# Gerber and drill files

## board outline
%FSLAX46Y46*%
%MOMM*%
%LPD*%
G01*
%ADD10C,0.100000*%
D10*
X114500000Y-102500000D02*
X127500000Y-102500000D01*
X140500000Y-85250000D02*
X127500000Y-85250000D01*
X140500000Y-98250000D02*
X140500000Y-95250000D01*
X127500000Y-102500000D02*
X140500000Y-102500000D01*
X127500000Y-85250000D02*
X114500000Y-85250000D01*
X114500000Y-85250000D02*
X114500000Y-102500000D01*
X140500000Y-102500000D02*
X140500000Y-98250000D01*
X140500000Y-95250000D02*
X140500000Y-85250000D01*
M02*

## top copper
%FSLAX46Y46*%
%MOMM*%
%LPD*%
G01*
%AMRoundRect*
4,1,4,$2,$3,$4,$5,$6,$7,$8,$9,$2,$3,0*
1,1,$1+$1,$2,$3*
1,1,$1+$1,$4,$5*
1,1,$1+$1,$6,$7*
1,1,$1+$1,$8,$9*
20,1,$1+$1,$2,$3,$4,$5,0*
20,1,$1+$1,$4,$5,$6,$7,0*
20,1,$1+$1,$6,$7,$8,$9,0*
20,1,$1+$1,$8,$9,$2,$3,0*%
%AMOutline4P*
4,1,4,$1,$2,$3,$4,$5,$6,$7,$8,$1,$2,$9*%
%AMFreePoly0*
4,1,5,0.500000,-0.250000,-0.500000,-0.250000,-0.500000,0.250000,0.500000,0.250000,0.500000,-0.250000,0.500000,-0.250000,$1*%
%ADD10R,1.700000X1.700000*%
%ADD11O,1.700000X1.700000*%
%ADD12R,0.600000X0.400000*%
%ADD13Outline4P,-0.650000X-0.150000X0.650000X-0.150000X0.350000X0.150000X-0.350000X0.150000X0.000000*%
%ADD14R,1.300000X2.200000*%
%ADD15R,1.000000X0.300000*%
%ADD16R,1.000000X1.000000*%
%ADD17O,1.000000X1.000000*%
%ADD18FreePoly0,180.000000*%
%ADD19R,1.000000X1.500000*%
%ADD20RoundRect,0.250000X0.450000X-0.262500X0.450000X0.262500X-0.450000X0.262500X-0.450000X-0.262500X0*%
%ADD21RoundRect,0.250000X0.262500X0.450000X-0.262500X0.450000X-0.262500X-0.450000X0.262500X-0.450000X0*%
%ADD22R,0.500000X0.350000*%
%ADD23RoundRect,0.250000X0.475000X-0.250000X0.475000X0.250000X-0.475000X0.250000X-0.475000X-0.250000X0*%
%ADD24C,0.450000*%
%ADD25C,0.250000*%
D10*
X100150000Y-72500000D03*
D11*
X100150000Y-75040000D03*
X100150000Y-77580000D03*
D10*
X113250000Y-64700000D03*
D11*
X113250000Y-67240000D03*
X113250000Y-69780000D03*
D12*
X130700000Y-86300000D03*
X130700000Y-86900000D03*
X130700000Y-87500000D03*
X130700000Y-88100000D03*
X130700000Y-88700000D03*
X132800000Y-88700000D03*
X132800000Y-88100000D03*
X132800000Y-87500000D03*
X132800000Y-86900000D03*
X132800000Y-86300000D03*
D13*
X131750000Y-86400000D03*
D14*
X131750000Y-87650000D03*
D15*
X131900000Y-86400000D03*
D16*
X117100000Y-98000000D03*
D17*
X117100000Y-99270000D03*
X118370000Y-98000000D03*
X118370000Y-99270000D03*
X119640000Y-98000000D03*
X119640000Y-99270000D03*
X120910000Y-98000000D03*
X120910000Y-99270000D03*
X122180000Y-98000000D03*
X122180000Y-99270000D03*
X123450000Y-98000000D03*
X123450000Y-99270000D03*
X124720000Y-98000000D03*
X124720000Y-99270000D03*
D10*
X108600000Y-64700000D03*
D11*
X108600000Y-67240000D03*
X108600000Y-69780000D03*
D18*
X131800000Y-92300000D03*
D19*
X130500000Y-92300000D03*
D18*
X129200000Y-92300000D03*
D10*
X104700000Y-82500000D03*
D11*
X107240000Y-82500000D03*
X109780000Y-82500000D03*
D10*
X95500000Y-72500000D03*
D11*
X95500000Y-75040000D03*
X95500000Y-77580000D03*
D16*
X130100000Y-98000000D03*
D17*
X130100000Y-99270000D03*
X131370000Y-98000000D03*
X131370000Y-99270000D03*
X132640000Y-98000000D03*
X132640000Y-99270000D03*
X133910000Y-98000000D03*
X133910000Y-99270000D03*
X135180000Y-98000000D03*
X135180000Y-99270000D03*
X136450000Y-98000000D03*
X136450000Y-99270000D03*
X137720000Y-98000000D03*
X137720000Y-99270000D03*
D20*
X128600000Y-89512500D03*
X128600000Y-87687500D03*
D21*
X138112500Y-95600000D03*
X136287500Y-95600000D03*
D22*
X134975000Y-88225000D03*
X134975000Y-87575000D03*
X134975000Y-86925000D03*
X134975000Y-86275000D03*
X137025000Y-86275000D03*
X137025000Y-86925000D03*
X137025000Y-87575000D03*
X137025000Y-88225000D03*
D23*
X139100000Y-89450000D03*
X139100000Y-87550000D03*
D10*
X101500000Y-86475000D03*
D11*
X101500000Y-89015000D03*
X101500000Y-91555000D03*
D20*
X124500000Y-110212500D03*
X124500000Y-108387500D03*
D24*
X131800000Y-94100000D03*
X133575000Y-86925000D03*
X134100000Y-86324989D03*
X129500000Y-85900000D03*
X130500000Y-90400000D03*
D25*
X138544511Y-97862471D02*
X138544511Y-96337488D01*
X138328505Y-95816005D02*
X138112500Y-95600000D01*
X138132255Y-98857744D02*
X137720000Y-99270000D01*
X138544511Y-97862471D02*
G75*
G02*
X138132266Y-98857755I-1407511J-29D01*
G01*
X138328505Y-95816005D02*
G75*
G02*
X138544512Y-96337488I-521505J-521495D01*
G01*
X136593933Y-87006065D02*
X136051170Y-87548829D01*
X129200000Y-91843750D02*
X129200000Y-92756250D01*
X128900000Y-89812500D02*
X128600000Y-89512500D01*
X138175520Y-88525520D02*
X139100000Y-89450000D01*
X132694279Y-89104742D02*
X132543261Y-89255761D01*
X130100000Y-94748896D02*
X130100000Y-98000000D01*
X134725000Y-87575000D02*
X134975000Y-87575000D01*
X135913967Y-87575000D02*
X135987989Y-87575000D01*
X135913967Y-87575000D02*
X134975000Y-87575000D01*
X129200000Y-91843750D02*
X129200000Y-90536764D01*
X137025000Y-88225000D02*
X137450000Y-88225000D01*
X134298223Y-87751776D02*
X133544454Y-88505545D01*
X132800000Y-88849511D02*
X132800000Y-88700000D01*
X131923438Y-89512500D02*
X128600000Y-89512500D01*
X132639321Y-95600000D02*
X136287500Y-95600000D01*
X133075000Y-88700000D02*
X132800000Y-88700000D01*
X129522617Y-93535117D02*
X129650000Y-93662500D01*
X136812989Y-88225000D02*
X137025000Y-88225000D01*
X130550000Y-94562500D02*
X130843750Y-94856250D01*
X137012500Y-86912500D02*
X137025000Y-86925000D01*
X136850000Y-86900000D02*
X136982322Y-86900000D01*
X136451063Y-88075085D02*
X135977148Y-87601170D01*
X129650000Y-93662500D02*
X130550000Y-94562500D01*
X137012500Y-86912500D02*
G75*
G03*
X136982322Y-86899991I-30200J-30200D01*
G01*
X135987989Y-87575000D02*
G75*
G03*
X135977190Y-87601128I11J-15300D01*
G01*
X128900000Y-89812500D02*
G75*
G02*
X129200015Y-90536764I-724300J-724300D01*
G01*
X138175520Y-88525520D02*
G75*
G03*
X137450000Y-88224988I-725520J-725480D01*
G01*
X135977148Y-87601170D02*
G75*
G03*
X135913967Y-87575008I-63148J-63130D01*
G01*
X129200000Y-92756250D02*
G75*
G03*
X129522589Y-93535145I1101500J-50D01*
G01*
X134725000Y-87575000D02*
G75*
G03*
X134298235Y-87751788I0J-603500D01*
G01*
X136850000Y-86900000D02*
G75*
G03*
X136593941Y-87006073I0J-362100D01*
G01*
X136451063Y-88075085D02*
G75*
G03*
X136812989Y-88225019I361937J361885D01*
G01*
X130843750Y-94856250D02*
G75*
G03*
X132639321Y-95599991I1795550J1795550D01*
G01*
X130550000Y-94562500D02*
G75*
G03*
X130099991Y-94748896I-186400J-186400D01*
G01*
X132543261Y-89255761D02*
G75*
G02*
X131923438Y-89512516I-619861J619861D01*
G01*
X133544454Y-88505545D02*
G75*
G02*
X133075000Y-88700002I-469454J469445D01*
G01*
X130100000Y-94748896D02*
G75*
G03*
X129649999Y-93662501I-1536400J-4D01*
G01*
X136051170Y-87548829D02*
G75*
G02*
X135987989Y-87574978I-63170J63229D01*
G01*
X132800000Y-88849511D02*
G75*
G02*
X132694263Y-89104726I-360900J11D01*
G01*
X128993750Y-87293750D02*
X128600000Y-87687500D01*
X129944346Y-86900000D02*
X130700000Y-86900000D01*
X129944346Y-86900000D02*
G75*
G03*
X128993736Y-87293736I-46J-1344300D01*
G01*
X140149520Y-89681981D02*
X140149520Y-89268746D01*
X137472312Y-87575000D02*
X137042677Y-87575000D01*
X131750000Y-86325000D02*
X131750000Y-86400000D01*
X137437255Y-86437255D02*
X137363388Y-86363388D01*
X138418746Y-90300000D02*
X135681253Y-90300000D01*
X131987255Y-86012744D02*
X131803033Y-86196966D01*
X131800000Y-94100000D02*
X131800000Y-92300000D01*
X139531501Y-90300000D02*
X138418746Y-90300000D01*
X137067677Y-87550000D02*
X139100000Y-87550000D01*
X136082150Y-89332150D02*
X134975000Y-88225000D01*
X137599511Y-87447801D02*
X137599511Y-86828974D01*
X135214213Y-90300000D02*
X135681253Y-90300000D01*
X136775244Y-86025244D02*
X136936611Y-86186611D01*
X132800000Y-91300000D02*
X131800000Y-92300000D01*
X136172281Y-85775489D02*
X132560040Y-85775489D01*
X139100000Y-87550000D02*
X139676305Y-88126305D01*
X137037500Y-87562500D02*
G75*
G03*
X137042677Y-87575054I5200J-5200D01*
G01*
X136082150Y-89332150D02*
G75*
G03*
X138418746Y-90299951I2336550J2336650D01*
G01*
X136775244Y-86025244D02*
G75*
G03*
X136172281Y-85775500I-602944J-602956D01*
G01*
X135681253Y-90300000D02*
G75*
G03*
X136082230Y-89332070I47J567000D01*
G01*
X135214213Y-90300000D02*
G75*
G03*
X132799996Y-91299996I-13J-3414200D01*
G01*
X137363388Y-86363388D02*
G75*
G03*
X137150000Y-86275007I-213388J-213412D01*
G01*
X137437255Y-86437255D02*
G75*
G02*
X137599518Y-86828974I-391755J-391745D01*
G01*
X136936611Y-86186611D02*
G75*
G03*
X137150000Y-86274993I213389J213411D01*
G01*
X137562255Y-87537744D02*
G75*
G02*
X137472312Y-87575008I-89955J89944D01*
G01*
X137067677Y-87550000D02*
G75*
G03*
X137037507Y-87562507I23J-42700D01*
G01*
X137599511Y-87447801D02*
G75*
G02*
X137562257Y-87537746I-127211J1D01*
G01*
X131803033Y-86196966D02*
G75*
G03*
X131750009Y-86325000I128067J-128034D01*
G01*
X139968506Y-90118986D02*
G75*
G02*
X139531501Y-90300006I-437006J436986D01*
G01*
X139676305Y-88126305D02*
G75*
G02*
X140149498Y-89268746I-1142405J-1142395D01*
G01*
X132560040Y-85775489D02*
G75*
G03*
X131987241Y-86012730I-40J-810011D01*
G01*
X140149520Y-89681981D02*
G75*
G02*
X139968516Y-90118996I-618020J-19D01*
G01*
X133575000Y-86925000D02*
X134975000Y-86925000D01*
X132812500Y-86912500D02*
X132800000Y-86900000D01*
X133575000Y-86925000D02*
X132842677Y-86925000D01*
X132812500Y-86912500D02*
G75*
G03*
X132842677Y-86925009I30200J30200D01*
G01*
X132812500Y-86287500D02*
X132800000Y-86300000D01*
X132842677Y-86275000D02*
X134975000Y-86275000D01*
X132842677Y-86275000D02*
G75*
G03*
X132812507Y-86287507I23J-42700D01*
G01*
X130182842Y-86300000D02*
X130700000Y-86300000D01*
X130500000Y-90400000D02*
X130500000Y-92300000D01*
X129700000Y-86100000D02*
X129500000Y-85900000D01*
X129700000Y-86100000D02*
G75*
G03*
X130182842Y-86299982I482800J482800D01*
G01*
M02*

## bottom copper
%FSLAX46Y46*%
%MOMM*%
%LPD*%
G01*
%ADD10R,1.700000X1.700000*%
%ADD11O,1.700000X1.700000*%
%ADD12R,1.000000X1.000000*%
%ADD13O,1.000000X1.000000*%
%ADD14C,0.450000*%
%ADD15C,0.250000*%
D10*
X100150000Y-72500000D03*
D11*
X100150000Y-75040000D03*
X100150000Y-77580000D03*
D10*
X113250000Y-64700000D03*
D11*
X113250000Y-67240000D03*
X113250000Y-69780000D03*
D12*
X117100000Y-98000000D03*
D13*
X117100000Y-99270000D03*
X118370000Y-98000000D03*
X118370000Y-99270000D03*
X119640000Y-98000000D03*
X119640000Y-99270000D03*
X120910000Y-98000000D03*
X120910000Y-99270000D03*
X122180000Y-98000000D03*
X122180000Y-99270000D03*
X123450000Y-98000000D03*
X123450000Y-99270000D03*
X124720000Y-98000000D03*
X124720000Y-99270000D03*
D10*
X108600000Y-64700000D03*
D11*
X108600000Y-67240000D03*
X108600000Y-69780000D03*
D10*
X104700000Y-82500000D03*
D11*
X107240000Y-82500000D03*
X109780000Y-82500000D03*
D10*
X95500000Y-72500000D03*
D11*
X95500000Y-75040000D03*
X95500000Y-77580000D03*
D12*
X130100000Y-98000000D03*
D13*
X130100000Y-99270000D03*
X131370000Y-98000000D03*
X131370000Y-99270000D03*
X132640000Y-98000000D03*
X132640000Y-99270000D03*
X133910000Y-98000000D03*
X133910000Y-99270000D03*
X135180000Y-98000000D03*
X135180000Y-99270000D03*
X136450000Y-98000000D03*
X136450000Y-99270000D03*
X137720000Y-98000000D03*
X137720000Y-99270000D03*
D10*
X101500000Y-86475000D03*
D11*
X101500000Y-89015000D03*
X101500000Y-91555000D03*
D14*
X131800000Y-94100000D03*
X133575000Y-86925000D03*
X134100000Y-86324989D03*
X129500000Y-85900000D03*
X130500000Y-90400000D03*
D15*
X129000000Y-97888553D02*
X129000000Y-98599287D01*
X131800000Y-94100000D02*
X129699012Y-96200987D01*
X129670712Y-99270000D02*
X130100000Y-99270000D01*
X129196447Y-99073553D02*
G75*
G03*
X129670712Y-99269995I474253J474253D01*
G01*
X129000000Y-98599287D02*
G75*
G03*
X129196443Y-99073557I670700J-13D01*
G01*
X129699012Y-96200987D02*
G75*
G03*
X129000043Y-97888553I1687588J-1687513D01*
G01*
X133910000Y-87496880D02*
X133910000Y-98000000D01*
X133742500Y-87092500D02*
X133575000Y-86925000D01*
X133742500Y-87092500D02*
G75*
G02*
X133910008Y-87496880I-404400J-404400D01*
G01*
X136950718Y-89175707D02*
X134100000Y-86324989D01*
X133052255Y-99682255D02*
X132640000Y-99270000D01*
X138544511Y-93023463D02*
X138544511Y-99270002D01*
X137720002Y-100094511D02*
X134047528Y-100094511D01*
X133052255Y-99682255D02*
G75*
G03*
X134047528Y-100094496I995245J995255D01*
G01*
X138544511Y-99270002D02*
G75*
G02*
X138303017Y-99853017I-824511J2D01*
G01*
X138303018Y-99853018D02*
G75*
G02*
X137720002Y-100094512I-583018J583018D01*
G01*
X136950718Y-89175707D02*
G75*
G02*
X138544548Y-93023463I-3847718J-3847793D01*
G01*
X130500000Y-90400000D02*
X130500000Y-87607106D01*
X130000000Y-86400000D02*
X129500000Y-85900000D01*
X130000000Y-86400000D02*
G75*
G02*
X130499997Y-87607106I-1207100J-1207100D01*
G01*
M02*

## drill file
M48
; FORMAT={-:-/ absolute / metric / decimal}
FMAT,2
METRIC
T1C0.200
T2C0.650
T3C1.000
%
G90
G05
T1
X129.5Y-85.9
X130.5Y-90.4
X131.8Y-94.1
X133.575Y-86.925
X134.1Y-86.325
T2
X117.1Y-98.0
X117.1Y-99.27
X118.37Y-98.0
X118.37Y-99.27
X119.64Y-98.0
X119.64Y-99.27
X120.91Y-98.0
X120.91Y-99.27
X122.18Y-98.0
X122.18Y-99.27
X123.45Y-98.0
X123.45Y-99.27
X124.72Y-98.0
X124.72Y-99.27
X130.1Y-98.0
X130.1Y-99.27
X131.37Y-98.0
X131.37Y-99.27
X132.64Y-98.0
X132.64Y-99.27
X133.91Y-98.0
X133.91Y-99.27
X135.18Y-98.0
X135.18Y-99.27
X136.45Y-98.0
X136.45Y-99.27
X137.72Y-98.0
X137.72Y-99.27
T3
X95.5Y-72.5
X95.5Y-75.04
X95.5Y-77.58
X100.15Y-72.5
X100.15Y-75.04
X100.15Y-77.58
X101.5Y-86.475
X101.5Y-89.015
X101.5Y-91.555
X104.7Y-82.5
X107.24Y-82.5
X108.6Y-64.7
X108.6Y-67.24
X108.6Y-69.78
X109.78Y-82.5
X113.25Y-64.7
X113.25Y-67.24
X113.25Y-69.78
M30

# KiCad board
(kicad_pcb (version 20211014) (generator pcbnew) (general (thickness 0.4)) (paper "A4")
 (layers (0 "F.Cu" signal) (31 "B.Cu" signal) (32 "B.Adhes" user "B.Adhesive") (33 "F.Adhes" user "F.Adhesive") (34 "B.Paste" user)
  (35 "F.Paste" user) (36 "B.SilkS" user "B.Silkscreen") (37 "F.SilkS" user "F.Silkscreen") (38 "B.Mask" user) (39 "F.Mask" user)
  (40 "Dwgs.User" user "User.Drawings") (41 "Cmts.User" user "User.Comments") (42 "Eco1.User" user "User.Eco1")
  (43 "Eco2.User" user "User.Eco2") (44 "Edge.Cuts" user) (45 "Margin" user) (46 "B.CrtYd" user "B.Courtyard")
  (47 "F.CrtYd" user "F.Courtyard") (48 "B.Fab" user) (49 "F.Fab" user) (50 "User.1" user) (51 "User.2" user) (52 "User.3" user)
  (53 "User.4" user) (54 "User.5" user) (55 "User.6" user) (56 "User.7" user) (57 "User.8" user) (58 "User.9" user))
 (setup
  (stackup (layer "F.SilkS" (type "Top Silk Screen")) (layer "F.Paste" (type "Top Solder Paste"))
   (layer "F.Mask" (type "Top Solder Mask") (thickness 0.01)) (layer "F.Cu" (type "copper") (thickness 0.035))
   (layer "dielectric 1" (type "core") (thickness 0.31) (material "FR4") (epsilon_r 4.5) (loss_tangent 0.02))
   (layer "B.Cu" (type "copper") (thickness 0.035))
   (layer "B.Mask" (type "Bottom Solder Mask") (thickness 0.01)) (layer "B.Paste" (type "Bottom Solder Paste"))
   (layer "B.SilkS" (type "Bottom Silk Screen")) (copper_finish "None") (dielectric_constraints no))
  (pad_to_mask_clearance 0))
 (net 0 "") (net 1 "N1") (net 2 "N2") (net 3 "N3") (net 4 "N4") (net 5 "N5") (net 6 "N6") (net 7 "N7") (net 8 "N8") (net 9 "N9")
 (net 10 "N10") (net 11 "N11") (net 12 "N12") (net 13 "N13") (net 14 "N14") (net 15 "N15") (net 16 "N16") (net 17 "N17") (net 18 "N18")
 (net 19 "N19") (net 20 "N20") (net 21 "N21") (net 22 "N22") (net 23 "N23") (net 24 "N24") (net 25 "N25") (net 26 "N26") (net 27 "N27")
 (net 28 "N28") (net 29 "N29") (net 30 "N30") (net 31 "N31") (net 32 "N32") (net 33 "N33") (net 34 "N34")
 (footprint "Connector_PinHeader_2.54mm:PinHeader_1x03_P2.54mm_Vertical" (layer "F.Cu") (at 100.15 72.5)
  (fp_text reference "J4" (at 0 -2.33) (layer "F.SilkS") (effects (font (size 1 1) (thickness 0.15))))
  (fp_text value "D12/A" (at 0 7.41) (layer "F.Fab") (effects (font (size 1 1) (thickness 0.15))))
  (pad "1" thru_hole rect (at 0 0) (size 1.7 1.7) (drill 1) (layers *.Cu *.Mask) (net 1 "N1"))
  (pad "2" thru_hole oval (at 0 2.54) (size 1.7 1.7) (drill 1) (layers *.Cu *.Mask) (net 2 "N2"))
  (pad "3" thru_hole oval (at 0 5.08) (size 1.7 1.7) (drill 1) (layers *.Cu *.Mask) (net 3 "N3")))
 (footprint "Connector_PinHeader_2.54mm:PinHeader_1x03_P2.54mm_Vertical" (layer "F.Cu") (at 113.25 64.7)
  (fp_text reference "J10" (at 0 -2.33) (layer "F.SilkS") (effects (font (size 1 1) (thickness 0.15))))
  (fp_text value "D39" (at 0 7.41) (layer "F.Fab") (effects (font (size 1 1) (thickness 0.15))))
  (pad "1" thru_hole rect (at 0 0) (size 1.7 1.7) (drill 1) (layers *.Cu *.Mask) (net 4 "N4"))
  (pad "2" thru_hole oval (at 0 2.54) (size 1.7 1.7) (drill 1) (layers *.Cu *.Mask) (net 2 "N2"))
  (pad "3" thru_hole oval (at 0 5.08) (size 1.7 1.7) (drill 1) (layers *.Cu *.Mask) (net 3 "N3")))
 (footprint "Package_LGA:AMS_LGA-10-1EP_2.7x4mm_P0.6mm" (layer "F.Cu") (at 131.75 87.5)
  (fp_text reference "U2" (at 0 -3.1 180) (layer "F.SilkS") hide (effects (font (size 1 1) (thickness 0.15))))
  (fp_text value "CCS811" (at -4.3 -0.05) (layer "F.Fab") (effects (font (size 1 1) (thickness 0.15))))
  (pad "1" smd rect (at -1.05 -1.2) (size 0.6 0.4) (layers "F.Cu" "F.Paste" "F.Mask") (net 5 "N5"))
  (pad "2" smd rect (at -1.05 -0.6) (size 0.6 0.4) (layers "F.Cu" "F.Paste" "F.Mask") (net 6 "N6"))
  (pad "3" smd rect (at -1.05 0) (size 0.6 0.4) (layers "F.Cu" "F.Paste" "F.Mask") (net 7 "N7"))
  (pad "4" smd rect (at -1.05 0.6) (size 0.6 0.4) (layers "F.Cu" "F.Paste" "F.Mask") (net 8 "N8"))
  (pad "5" smd rect (at -1.05 1.2) (size 0.6 0.4) (layers "F.Cu" "F.Paste" "F.Mask") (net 8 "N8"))
  (pad "6" smd rect (at 1.05 1.2) (size 0.6 0.4) (layers "F.Cu" "F.Paste" "F.Mask") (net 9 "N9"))
  (pad "7" smd rect (at 1.05 0.6) (size 0.6 0.4) (layers "F.Cu" "F.Paste" "F.Mask") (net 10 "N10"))
  (pad "8" smd rect (at 1.05 0) (size 0.6 0.4) (layers "F.Cu" "F.Paste" "F.Mask") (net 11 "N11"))
  (pad "9" smd rect (at 1.05 -0.6) (size 0.6 0.4) (layers "F.Cu" "F.Paste" "F.Mask") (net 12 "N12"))
  (pad "10" smd rect (at 1.05 -1.2) (size 0.6 0.4) (layers "F.Cu" "F.Paste" "F.Mask") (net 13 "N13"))
  (pad "11" smd trapezoid (at 0 -1.1) (size 1 0.3) (rect_delta 0 0.3) (layers "F.Cu" "F.Paste" "F.Mask") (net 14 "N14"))
  (pad "11" smd rect (at 0 0.15) (size 1.3 2.2) (layers "F.Cu" "F.Paste" "F.Mask") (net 14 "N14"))
  (pad "11" smd rect (at 0.15 -1.1) (size 1 0.3) (layers "F.Cu" "F.Paste" "F.Mask") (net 14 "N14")))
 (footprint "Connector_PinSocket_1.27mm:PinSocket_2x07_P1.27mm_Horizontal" (layer "F.Cu") (at 117.1 98 90)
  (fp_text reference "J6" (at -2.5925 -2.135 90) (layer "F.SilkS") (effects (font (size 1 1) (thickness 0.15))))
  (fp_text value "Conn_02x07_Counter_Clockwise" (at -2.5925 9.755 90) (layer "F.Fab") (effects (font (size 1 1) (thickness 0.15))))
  (pad "1" thru_hole rect (at 0 0 90) (size 1 1) (drill 0.65) (layers *.Cu *.Mask) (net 2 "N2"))
  (pad "2" thru_hole oval (at -1.27 0 90) (size 1 1) (drill 0.65) (layers *.Cu *.Mask) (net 3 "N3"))
  (pad "3" thru_hole oval (at 0 1.27 90) (size 1 1) (drill 0.65) (layers *.Cu *.Mask) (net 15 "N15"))
  (pad "4" thru_hole oval (at -1.27 1.27 90) (size 1 1) (drill 0.65) (layers *.Cu *.Mask) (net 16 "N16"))
  (pad "5" thru_hole oval (at 0 2.54 90) (size 1 1) (drill 0.65) (layers *.Cu *.Mask) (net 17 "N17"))
  (pad "6" thru_hole oval (at -1.27 2.54 90) (size 1 1) (drill 0.65) (layers *.Cu *.Mask) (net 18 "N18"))
  (pad "7" thru_hole oval (at 0 3.81 90) (size 1 1) (drill 0.65) (layers *.Cu *.Mask) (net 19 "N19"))
  (pad "8" thru_hole oval (at -1.27 3.81 90) (size 1 1) (drill 0.65) (layers *.Cu *.Mask) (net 4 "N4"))
  (pad "9" thru_hole oval (at 0 5.08 90) (size 1 1) (drill 0.65) (layers *.Cu *.Mask) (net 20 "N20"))
  (pad "10" thru_hole oval (at -1.27 5.08 90) (size 1 1) (drill 0.65) (layers *.Cu *.Mask) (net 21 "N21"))
  (pad "11" thru_hole oval (at 0 6.35 90) (size 1 1) (drill 0.65) (layers *.Cu *.Mask) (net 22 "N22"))
  (pad "12" thru_hole oval (at -1.27 6.35 90) (size 1 1) (drill 0.65) (layers *.Cu *.Mask) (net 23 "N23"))
  (pad "13" thru_hole oval (at 0 7.62 90) (size 1 1) (drill 0.65) (layers *.Cu *.Mask) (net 1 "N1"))
  (pad "14" thru_hole oval (at -1.27 7.62 90) (size 1 1) (drill 0.65) (layers *.Cu *.Mask) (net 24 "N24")))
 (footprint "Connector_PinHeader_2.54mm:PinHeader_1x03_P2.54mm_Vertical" (layer "F.Cu") (at 108.6 64.7)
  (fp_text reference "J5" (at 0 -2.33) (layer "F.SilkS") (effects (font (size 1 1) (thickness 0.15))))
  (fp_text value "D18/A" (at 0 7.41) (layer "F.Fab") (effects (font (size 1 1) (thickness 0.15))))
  (pad "1" thru_hole rect (at 0 0) (size 1.7 1.7) (drill 1) (layers *.Cu *.Mask) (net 21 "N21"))
  (pad "2" thru_hole oval (at 0 2.54) (size 1.7 1.7) (drill 1) (layers *.Cu *.Mask) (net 2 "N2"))
  (pad "3" thru_hole oval (at 0 5.08) (size 1.7 1.7) (drill 1) (layers *.Cu *.Mask) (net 3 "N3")))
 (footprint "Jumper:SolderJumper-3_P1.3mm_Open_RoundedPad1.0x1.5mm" (layer "F.Cu") (at 130.5 92.3 180)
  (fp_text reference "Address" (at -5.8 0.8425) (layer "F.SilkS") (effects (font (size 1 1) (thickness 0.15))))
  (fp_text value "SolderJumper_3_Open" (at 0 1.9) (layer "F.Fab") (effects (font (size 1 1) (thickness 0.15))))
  (pad "1" smd custom (at -1.3 0 180) (size 1 0.5) (layers "F.Cu" "F.Mask") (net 14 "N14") (zone_connect 2)
   (options (clearance outline) (anchor rect)) (primitives))
  (pad "2" smd rect (at 0 0 180) (size 1 1.5) (layers "F.Cu" "F.Mask") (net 5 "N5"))
  (pad "3" smd custom (at 1.3 0 180) (size 1 0.5) (layers "F.Cu" "F.Mask") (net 9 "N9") (zone_connect 2)
   (options (clearance outline) (anchor rect)) (primitives)))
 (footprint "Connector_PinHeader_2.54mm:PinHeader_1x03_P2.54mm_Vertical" (layer "F.Cu") (at 104.7 82.5 90)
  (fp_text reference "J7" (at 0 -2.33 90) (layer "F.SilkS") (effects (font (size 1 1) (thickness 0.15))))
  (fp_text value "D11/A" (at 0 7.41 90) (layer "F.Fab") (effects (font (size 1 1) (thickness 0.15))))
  (pad "1" thru_hole rect (at 0 0 90) (size 1.7 1.7) (drill 1) (layers *.Cu *.Mask) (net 23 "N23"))
  (pad "2" thru_hole oval (at 0 2.54 90) (size 1.7 1.7) (drill 1) (layers *.Cu *.Mask) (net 2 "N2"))
  (pad "3" thru_hole oval (at 0 5.08 90) (size 1.7 1.7) (drill 1) (layers *.Cu *.Mask) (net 3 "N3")))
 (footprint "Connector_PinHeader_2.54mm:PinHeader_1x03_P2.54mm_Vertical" (layer "F.Cu") (at 95.5 72.5)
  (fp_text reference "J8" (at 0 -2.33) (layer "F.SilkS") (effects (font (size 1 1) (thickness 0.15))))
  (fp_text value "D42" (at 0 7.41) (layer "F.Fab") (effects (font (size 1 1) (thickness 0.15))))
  (pad "1" thru_hole rect (at 0 0) (size 1.7 1.7) (drill 1) (layers *.Cu *.Mask) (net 20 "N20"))
  (pad "2" thru_hole oval (at 0 2.54) (size 1.7 1.7) (drill 1) (layers *.Cu *.Mask) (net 2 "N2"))
  (pad "3" thru_hole oval (at 0 5.08) (size 1.7 1.7) (drill 1) (layers *.Cu *.Mask) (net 3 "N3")))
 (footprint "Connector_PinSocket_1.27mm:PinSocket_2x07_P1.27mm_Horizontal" (layer "F.Cu") (at 130.1 98 90)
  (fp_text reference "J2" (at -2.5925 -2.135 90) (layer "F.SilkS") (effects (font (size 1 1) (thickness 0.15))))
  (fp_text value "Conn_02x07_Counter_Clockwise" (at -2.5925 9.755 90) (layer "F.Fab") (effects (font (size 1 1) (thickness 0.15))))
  (pad "1" thru_hole rect (at 0 0 90) (size 1 1) (drill 0.65) (layers *.Cu *.Mask) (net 9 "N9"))
  (pad "2" thru_hole oval (at -1.27 0 90) (size 1 1) (drill 0.65) (layers *.Cu *.Mask) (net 14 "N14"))
  (pad "3" thru_hole oval (at 0 1.27 90) (size 1 1) (drill 0.65) (layers *.Cu *.Mask) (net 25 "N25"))
  (pad "4" thru_hole oval (at -1.27 1.27 90) (size 1 1) (drill 0.65) (layers *.Cu *.Mask) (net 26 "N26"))
  (pad "5" thru_hole oval (at 0 2.54 90) (size 1 1) (drill 0.65) (layers *.Cu *.Mask) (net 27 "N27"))
  (pad "6" thru_hole oval (at -1.27 2.54 90) (size 1 1) (drill 0.65) (layers *.Cu *.Mask) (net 13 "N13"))
  (pad "7" thru_hole oval (at 0 3.81 90) (size 1 1) (drill 0.65) (layers *.Cu *.Mask) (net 12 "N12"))
  (pad "8" thru_hole oval (at -1.27 3.81 90) (size 1 1) (drill 0.65) (layers *.Cu *.Mask) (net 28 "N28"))
  (pad "9" thru_hole oval (at 0 5.08 90) (size 1 1) (drill 0.65) (layers *.Cu *.Mask) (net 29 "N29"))
  (pad "10" thru_hole oval (at -1.27 5.08 90) (size 1 1) (drill 0.65) (layers *.Cu *.Mask) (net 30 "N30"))
  (pad "11" thru_hole oval (at 0 6.35 90) (size 1 1) (drill 0.65) (layers *.Cu *.Mask) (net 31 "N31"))
  (pad "12" thru_hole oval (at -1.27 6.35 90) (size 1 1) (drill 0.65) (layers *.Cu *.Mask) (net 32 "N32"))
  (pad "13" thru_hole oval (at 0 7.62 90) (size 1 1) (drill 0.65) (layers *.Cu *.Mask) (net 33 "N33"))
  (pad "14" thru_hole oval (at -1.27 7.62 90) (size 1 1) (drill 0.65) (layers *.Cu *.Mask) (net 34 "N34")))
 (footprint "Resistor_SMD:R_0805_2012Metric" (layer "F.Cu") (at 128.6 88.6 90)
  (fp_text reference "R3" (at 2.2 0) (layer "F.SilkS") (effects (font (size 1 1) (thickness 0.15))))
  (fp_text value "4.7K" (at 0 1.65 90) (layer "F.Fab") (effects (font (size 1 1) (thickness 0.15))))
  (pad "1" smd roundrect (at -0.9125 0 90) (size 1.025 1.4) (layers "F.Cu" "F.Paste" "F.Mask") (roundrect_rratio 0.243902) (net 9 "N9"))
  (pad "2" smd roundrect (at 0.9125 0 90) (size 1.025 1.4) (layers "F.Cu" "F.Paste" "F.Mask") (roundrect_rratio 0.243902) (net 6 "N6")))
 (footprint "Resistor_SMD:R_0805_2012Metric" (layer "F.Cu") (at 137.2 95.6 180)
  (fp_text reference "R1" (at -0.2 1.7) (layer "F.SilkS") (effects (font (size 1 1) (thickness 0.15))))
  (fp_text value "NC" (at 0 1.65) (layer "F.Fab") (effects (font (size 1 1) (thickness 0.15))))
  (pad "1" smd roundrect (at -0.9125 0 180) (size 1.025 1.4) (layers "F.Cu" "F.Paste" "F.Mask") (roundrect_rratio 0.243902) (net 34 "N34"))
  (pad "2" smd roundrect (at 0.9125 0 180) (size 1.025 1.4) (layers "F.Cu" "F.Paste" "F.Mask") (roundrect_rratio 0.243902) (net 9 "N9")))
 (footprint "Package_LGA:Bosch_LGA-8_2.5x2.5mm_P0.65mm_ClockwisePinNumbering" (layer "F.Cu") (at 136 87.25 90)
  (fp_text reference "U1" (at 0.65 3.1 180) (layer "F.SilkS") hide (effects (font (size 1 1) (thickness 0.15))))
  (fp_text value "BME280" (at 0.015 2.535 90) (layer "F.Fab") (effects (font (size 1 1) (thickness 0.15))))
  (pad "1" smd rect (at -0.975 -1.025 180) (size 0.5 0.35) (layers "F.Cu" "F.Paste" "F.Mask") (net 14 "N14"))
  (pad "2" smd rect (at -0.325 -1.025 180) (size 0.5 0.35) (layers "F.Cu" "F.Paste" "F.Mask") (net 9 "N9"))
  (pad "3" smd rect (at 0.325 -1.025 180) (size 0.5 0.35) (layers "F.Cu" "F.Paste" "F.Mask") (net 12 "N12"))
  (pad "4" smd rect (at 0.975 -1.025 180) (size 0.5 0.35) (layers "F.Cu" "F.Paste" "F.Mask") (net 13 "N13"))
  (pad "5" smd rect (at 0.975 1.025 180) (size 0.5 0.35) (layers "F.Cu" "F.Paste" "F.Mask") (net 14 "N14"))
  (pad "6" smd rect (at 0.325 1.025 180) (size 0.5 0.35) (layers "F.Cu" "F.Paste" "F.Mask") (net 9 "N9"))
  (pad "7" smd rect (at -0.325 1.025 180) (size 0.5 0.35) (layers "F.Cu" "F.Paste" "F.Mask") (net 14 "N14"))
  (pad "8" smd rect (at -0.975 1.025 180) (size 0.5 0.35) (layers "F.Cu" "F.Paste" "F.Mask") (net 9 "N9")))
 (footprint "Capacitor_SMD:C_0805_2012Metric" (layer "F.Cu") (at 139.1 88.5 90)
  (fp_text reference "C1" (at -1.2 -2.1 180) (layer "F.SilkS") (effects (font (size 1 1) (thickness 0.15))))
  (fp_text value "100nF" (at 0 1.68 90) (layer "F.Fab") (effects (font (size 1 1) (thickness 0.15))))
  (pad "1" smd roundrect (at -0.95 0 90) (size 1 1.45) (layers "F.Cu" "F.Paste" "F.Mask") (roundrect_rratio 0.25) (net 9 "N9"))
  (pad "2" smd roundrect (at 0.95 0 90) (size 1 1.45) (layers "F.Cu" "F.Paste" "F.Mask") (roundrect_rratio 0.25) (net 14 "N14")))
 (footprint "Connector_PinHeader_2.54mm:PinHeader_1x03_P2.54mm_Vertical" (layer "F.Cu") (at 101.5 86.475)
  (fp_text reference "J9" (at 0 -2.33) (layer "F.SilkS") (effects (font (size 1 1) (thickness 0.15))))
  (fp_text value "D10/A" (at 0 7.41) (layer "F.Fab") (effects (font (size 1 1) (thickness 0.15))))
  (pad "1" thru_hole rect (at 0 0) (size 1.7 1.7) (drill 1) (layers *.Cu *.Mask) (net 22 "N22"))
  (pad "2" thru_hole oval (at 0 2.54) (size 1.7 1.7) (drill 1) (layers *.Cu *.Mask) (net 2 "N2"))
  (pad "3" thru_hole oval (at 0 5.08) (size 1.7 1.7) (drill 1) (layers *.Cu *.Mask) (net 3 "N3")))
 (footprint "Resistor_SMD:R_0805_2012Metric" (layer "F.Cu") (at 124.5 109.3 90)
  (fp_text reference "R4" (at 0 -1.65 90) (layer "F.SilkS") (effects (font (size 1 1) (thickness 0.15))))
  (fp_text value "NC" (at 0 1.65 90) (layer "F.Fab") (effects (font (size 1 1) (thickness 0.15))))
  (pad "1" smd roundrect (at -0.9125 0 90) (size 1.025 1.4) (layers "F.Cu" "F.Paste" "F.Mask") (roundrect_rratio 0.243902) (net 24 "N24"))
  (pad "2" smd roundrect (at 0.9125 0 90) (size 1.025 1.4) (layers "F.Cu" "F.Paste" "F.Mask") (roundrect_rratio 0.243902) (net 2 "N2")))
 (gr_line (start 114.5 102.5) (end 127.5 102.5) (layer "Edge.Cuts") (width 0.1))
 (gr_line (start 140.5 85.25) (end 127.5 85.25) (layer "Edge.Cuts") (width 0.1))
 (gr_line (start 140.5 98.25) (end 140.5 95.25) (layer "Edge.Cuts") (width 0.1))
 (gr_line (start 127.5 102.5) (end 140.5 102.5) (layer "Edge.Cuts") (width 0.1))
 (gr_line (start 127.5 85.25) (end 114.5 85.25) (layer "Edge.Cuts") (width 0.1))
 (gr_line (start 114.5 85.25) (end 114.5 102.5) (layer "Edge.Cuts") (width 0.1))
 (gr_line (start 140.5 102.5) (end 140.5 98.25) (layer "Edge.Cuts") (width 0.1))
 (gr_line (start 140.5 95.25) (end 140.5 85.25) (layer "Edge.Cuts") (width 0.1))
 (segment (start 138.544511 97.862471) (end 138.544511 96.337488) (width 0.25) (layer "F.Cu") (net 34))
 (segment (start 138.328505 95.816005) (end 138.1125 95.6) (width 0.25) (layer "F.Cu") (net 34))
 (segment (start 138.132255 98.857744) (end 137.72 99.27) (width 0.25) (layer "F.Cu") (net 34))
 (arc (start 138.544511 97.862471) (mid 138.437369 98.401109) (end 138.132255 98.857744) (width 0.25) (layer "F.Cu") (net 34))
 (arc (start 138.328505 95.816005) (mid 138.488372 96.055263) (end 138.544511 96.337488) (width 0.25) (layer "F.Cu") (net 34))
 (segment (start 136.593933 87.006065) (end 136.05117 87.548829) (width 0.25) (layer "F.Cu") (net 9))
 (segment (start 129.2 91.84375) (end 129.2 92.75625) (width 0.25) (layer "F.Cu") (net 9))
 (segment (start 128.9 89.8125) (end 128.6 89.5125) (width 0.25) (layer "F.Cu") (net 9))
 (segment (start 138.17552 88.52552) (end 139.1 89.45) (width 0.25) (layer "F.Cu") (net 9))
 (segment (start 132.694279 89.104742) (end 132.543261 89.255761) (width 0.25) (layer "F.Cu") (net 9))
 (segment (start 130.1 94.748896) (end 130.1 98) (width 0.25) (layer "F.Cu") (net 9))
 (segment (start 134.725 87.575) (end 134.975 87.575) (width 0.25) (layer "F.Cu") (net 9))
 (segment (start 135.913967 87.575) (end 135.987989 87.575) (width 0.25) (layer "F.Cu") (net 9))
 (segment (start 135.913967 87.575) (end 134.975 87.575) (width 0.25) (layer "F.Cu") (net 9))
 (segment (start 129.2 91.84375) (end 129.2 90.536764) (width 0.25) (layer "F.Cu") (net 9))
 (segment (start 137.025 88.225) (end 137.45 88.225) (width 0.25) (layer "F.Cu") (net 9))
 (segment (start 134.298223 87.751776) (end 133.544454 88.505545) (width 0.25) (layer "F.Cu") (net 9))
 (segment (start 132.8 88.849511) (end 132.8 88.7) (width 0.25) (layer "F.Cu") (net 9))
 (segment (start 131.923438 89.5125) (end 128.6 89.5125) (width 0.25) (layer "F.Cu") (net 9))
 (segment (start 132.639321 95.6) (end 136.2875 95.6) (width 0.25) (layer "F.Cu") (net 9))
 (segment (start 133.075 88.7) (end 132.8 88.7) (width 0.25) (layer "F.Cu") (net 9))
 (segment (start 129.522617 93.535117) (end 129.65 93.6625) (width 0.25) (layer "F.Cu") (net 9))
 (segment (start 136.812989 88.225) (end 137.025 88.225) (width 0.25) (layer "F.Cu") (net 9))
 (segment (start 130.55 94.5625) (end 130.84375 94.85625) (width 0.25) (layer "F.Cu") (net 9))
 (segment (start 137.0125 86.9125) (end 137.025 86.925) (width 0.25) (layer "F.Cu") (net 9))
 (segment (start 136.85 86.9) (end 136.982322 86.9) (width 0.25) (layer "F.Cu") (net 9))
 (segment (start 136.451063 88.075085) (end 135.977148 87.60117) (width 0.25) (layer "F.Cu") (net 9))
 (segment (start 129.65 93.6625) (end 130.55 94.5625) (width 0.25) (layer "F.Cu") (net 9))
 (arc (start 137.0125 86.9125) (mid 136.998654 86.903248) (end 136.982322 86.9) (width 0.25) (layer "F.Cu") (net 9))
 (arc (start 135.987989 87.575) (mid 135.973825 87.584463) (end 135.977148 87.60117) (width 0.25) (layer "F.Cu") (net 9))
 (arc (start 128.9 89.8125) (mid 129.122032 90.144795) (end 129.2 90.536764) (width 0.25) (layer "F.Cu") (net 9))
 (arc (start 138.17552 88.52552) (mid 137.842648 88.303102) (end 137.45 88.225) (width 0.25) (layer "F.Cu") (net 9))
 (arc (start 135.977148 87.60117) (mid 135.94816 87.581801) (end 135.913967 87.575) (width 0.25) (layer "F.Cu") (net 9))
 (arc (start 129.2 92.75625) (mid 129.283845 93.177769) (end 129.522617 93.535117) (width 0.25) (layer "F.Cu") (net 9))
 (arc (start 134.725 87.575) (mid 134.49403 87.620942) (end 134.298223 87.751776) (width 0.25) (layer "F.Cu") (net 9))
 (arc (start 136.85 86.9) (mid 136.711417 86.927565) (end 136.593933 87.006065) (width 0.25) (layer "F.Cu") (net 9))
 (arc (start 136.451063 88.075085) (mid 136.617116 88.186038) (end 136.812989 88.225) (width 0.25) (layer "F.Cu") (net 9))
 (arc (start 130.84375 94.85625) (mid 131.667565 95.406705) (end 132.639321 95.6) (width 0.25) (layer "F.Cu") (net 9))
 (arc (start 130.55 94.5625) (mid 130.262727 94.505357) (end 130.1 94.748896) (width 0.25) (layer "F.Cu") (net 9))
 (arc (start 132.543261 89.255761) (mid 132.258883 89.445775) (end 131.923438 89.5125) (width 0.25) (layer "F.Cu") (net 9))
 (arc (start 133.544454 88.505545) (mid 133.329066 88.649462) (end 133.075 88.7) (width 0.25) (layer "F.Cu") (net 9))
 (arc (start 130.1 94.748896) (mid 129.983048 94.160942) (end 129.65 93.6625) (width 0.25) (layer "F.Cu") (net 9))
 (arc (start 136.05117 87.548829) (mid 136.022182 87.568198) (end 135.987989 87.575) (width 0.25) (layer "F.Cu") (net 9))
 (arc (start 132.8 88.849511) (mid 132.772524 88.987641) (end 132.694279 89.104742) (width 0.25) (layer "F.Cu") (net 9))
 (segment (start 128.99375 87.29375) (end 128.6 87.6875) (width 0.25) (layer "F.Cu") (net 6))
 (segment (start 129.944346 86.9) (end 130.7 86.9) (width 0.25) (layer "F.Cu") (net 6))
 (arc (start 129.944346 86.9) (mid 129.429887 87.002332) (end 128.99375 87.29375) (width 0.25) (layer "F.Cu") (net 6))
 (segment (start 140.14952 89.681981) (end 140.14952 89.268746) (width 0.25) (layer "F.Cu") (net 14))
 (segment (start 137.472312 87.575) (end 137.042677 87.575) (width 0.25) (layer "F.Cu") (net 14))
 (segment (start 131.75 86.325) (end 131.75 86.4) (width 0.25) (layer "F.Cu") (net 14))
 (segment (start 137.437255 86.437255) (end 137.363388 86.363388) (width 0.25) (layer "F.Cu") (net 14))
 (segment (start 138.418746 90.3) (end 135.681253 90.3) (width 0.25) (layer "F.Cu") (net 14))
 (segment (start 131.987255 86.012744) (end 131.803033 86.196966) (width 0.25) (layer "F.Cu") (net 14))
 (segment (start 131.8 94.1) (end 131.8 92.3) (width 0.25) (layer "F.Cu") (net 14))
 (segment (start 139.531501 90.3) (end 138.418746 90.3) (width 0.25) (layer "F.Cu") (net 14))
 (segment (start 137.067677 87.55) (end 139.1 87.55) (width 0.25) (layer "F.Cu") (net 14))
 (segment (start 136.08215 89.33215) (end 134.975 88.225) (width 0.25) (layer "F.Cu") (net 14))
 (segment (start 137.599511 87.447801) (end 137.599511 86.828974) (width 0.25) (layer "F.Cu") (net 14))
 (segment (start 135.214213 90.3) (end 135.681253 90.3) (width 0.25) (layer "F.Cu") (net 14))
 (segment (start 136.775244 86.025244) (end 136.936611 86.186611) (width 0.25) (layer "F.Cu") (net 14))
 (segment (start 132.8 91.3) (end 131.8 92.3) (width 0.25) (layer "F.Cu") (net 14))
 (segment (start 136.172281 85.775489) (end 132.56004 85.775489) (width 0.25) (layer "F.Cu") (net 14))
 (segment (start 139.1 87.55) (end 139.676305 88.126305) (width 0.25) (layer "F.Cu") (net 14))
 (via (at 131.8 94.1) (size 0.45) (drill 0.2) (layers "F.Cu" "B.Cu") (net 14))
 (arc (start 137.0375 87.5625) (mid 137.035912 87.570479) (end 137.042677 87.575) (width 0.25) (layer "F.Cu") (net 14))
 (arc (start 136.08215 89.33215) (mid 137.154189 90.048463) (end 138.418746 90.3) (width 0.25) (layer "F.Cu") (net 14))
 (arc (start 136.775244 86.025244) (mid 136.498602 85.840398) (end 136.172281 85.775489) (width 0.25) (layer "F.Cu") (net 14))
 (arc (start 135.681253 90.3) (mid 136.205049 89.95001) (end 136.08215 89.33215) (width 0.25) (layer "F.Cu") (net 14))
 (arc (start 135.214213 90.3) (mid 133.90765 90.559891) (end 132.8 91.3) (width 0.25) (layer "F.Cu") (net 14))
 (arc (start 137.363388 86.363388) (mid 137.265484 86.297971) (end 137.15 86.275) (width 0.25) (layer "F.Cu") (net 14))
 (arc (start 137.437255 86.437255) (mid 137.557342 86.616977) (end 137.599511 86.828974) (width 0.25) (layer "F.Cu") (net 14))
 (arc (start 136.936611 86.186611) (mid 137.034514 86.252028) (end 137.15 86.275) (width 0.25) (layer "F.Cu") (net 14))
 (arc (start 137.562255 87.537744) (mid 137.520989 87.565317) (end 137.472312 87.575) (width 0.25) (layer "F.Cu") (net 14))
 (arc (start 137.067677 87.55) (mid 137.051345 87.553248) (end 137.0375 87.5625) (width 0.25) (layer "F.Cu") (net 14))
 (arc (start 137.599511 87.447801) (mid 137.589828 87.496478) (end 137.562255 87.537744) (width 0.25) (layer "F.Cu") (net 14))
 (arc (start 131.803033 86.196966) (mid 131.763782 86.255708) (end 131.75 86.325) (width 0.25) (layer "F.Cu") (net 14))
 (arc (start 139.968506 90.118986) (mid 139.768006 90.252955) (end 139.531501 90.3) (width 0.25) (layer "F.Cu") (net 14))
 (arc (start 139.676305 88.126305) (mid 140.026535 88.650461) (end 140.14952 89.268746) (width 0.25) (layer "F.Cu") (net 14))
 (arc (start 132.56004 85.775489) (mid 132.250051 85.837149) (end 131.987255 86.012744) (width 0.25) (layer "F.Cu") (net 14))
 (arc (start 140.14952 89.681981) (mid 140.102475 89.918486) (end 139.968506 90.118986) (width 0.25) (layer "F.Cu") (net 14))
 (segment (start 129 97.888553) (end 129 98.599287) (width 0.25) (layer "B.Cu") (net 14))
 (segment (start 131.8 94.1) (end 129.699012 96.200987) (width 0.25) (layer "B.Cu") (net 14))
 (segment (start 129.670712 99.27) (end 130.1 99.27) (width 0.25) (layer "B.Cu") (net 14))
 (arc (start 129.196447 99.073553) (mid 129.414041 99.218945) (end 129.670712 99.27) (width 0.25) (layer "B.Cu") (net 14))
 (arc (start 129 98.599287) (mid 129.051054 98.855958) (end 129.196447 99.073553) (width 0.25) (layer "B.Cu") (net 14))
 (arc (start 129.699012 96.200987) (mid 129.181667 96.975248) (end 129 97.888553) (width 0.25) (layer "B.Cu") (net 14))
 (segment (start 133.575 86.925) (end 134.975 86.925) (width 0.25) (layer "F.Cu") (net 12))
 (segment (start 132.8125 86.9125) (end 132.8 86.9) (width 0.25) (layer "F.Cu") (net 12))
 (segment (start 133.575 86.925) (end 132.842677 86.925) (width 0.25) (layer "F.Cu") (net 12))
 (via (at 133.575 86.925) (size 0.45) (drill 0.2) (layers "F.Cu" "B.Cu") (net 12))
 (arc (start 132.8125 86.9125) (mid 132.826345 86.921751) (end 132.842677 86.925) (width 0.25) (layer "F.Cu") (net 12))
 (segment (start 133.91 87.49688) (end 133.91 98) (width 0.25) (layer "B.Cu") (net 12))
 (segment (start 133.7425 87.0925) (end 133.575 86.925) (width 0.25) (layer "B.Cu") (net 12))
 (arc (start 133.7425 87.0925) (mid 133.866468 87.278031) (end 133.91 87.49688) (width 0.25) (layer "B.Cu") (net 12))
 (segment (start 132.8125 86.2875) (end 132.8 86.3) (width 0.25) (layer "F.Cu") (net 13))
 (segment (start 132.842677 86.275) (end 134.975 86.275) (width 0.25) (layer "F.Cu") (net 13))
 (via (at 134.1 86.324989) (size 0.45) (drill 0.2) (layers "F.Cu" "B.Cu") (free) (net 13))
 (arc (start 132.842677 86.275) (mid 132.826345 86.278248) (end 132.8125 86.2875) (width 0.25) (layer "F.Cu") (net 13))
 (segment (start 136.950718 89.175707) (end 134.1 86.324989) (width 0.25) (layer "B.Cu") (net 13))
 (segment (start 133.052255 99.682255) (end 132.64 99.27) (width 0.25) (layer "B.Cu") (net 13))
 (segment (start 138.544511 93.023463) (end 138.544511 99.270002) (width 0.25) (layer "B.Cu") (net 13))
 (segment (start 137.720002 100.094511) (end 134.047528 100.094511) (width 0.25) (layer "B.Cu") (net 13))
 (arc (start 133.052255 99.682255) (mid 133.50889 99.987369) (end 134.047528 100.094511) (width 0.25) (layer "B.Cu") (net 13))
 (arc (start 138.544511 99.270002) (mid 138.481749 99.585528) (end 138.303018 99.853018) (width 0.25) (layer "B.Cu") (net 13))
 (arc (start 138.303018 99.853018) (mid 138.035528 100.031749) (end 137.720002 100.094511) (width 0.25) (layer "B.Cu") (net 13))
 (arc (start 136.950718 89.175707) (mid 138.130297 90.941072) (end 138.544511 93.023463) (width 0.25) (layer "B.Cu") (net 13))
 (segment (start 130.182842 86.3) (end 130.7 86.3) (width 0.25) (layer "F.Cu") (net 5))
 (segment (start 130.5 90.4) (end 130.5 92.3) (width 0.25) (layer "F.Cu") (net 5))
 (segment (start 129.7 86.1) (end 129.5 85.9) (width 0.25) (layer "F.Cu") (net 5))
 (via (at 129.5 85.9) (size 0.45) (drill 0.2) (layers "F.Cu" "B.Cu") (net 5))
 (via (at 130.5 90.4) (size 0.45) (drill 0.2) (layers "F.Cu" "B.Cu") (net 5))
 (arc (start 129.7 86.1) (mid 129.921529 86.248021) (end 130.182842 86.3) (width 0.25) (layer "F.Cu") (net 5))
 (segment (start 130.5 90.4) (end 130.5 87.607106) (width 0.25) (layer "B.Cu") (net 5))
 (segment (start 130 86.4) (end 129.5 85.9) (width 0.25) (layer "B.Cu") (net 5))
 (arc (start 130 86.4) (mid 130.370054 86.953825) (end 130.5 87.607106) (width 0.25) (layer "B.Cu") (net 5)))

